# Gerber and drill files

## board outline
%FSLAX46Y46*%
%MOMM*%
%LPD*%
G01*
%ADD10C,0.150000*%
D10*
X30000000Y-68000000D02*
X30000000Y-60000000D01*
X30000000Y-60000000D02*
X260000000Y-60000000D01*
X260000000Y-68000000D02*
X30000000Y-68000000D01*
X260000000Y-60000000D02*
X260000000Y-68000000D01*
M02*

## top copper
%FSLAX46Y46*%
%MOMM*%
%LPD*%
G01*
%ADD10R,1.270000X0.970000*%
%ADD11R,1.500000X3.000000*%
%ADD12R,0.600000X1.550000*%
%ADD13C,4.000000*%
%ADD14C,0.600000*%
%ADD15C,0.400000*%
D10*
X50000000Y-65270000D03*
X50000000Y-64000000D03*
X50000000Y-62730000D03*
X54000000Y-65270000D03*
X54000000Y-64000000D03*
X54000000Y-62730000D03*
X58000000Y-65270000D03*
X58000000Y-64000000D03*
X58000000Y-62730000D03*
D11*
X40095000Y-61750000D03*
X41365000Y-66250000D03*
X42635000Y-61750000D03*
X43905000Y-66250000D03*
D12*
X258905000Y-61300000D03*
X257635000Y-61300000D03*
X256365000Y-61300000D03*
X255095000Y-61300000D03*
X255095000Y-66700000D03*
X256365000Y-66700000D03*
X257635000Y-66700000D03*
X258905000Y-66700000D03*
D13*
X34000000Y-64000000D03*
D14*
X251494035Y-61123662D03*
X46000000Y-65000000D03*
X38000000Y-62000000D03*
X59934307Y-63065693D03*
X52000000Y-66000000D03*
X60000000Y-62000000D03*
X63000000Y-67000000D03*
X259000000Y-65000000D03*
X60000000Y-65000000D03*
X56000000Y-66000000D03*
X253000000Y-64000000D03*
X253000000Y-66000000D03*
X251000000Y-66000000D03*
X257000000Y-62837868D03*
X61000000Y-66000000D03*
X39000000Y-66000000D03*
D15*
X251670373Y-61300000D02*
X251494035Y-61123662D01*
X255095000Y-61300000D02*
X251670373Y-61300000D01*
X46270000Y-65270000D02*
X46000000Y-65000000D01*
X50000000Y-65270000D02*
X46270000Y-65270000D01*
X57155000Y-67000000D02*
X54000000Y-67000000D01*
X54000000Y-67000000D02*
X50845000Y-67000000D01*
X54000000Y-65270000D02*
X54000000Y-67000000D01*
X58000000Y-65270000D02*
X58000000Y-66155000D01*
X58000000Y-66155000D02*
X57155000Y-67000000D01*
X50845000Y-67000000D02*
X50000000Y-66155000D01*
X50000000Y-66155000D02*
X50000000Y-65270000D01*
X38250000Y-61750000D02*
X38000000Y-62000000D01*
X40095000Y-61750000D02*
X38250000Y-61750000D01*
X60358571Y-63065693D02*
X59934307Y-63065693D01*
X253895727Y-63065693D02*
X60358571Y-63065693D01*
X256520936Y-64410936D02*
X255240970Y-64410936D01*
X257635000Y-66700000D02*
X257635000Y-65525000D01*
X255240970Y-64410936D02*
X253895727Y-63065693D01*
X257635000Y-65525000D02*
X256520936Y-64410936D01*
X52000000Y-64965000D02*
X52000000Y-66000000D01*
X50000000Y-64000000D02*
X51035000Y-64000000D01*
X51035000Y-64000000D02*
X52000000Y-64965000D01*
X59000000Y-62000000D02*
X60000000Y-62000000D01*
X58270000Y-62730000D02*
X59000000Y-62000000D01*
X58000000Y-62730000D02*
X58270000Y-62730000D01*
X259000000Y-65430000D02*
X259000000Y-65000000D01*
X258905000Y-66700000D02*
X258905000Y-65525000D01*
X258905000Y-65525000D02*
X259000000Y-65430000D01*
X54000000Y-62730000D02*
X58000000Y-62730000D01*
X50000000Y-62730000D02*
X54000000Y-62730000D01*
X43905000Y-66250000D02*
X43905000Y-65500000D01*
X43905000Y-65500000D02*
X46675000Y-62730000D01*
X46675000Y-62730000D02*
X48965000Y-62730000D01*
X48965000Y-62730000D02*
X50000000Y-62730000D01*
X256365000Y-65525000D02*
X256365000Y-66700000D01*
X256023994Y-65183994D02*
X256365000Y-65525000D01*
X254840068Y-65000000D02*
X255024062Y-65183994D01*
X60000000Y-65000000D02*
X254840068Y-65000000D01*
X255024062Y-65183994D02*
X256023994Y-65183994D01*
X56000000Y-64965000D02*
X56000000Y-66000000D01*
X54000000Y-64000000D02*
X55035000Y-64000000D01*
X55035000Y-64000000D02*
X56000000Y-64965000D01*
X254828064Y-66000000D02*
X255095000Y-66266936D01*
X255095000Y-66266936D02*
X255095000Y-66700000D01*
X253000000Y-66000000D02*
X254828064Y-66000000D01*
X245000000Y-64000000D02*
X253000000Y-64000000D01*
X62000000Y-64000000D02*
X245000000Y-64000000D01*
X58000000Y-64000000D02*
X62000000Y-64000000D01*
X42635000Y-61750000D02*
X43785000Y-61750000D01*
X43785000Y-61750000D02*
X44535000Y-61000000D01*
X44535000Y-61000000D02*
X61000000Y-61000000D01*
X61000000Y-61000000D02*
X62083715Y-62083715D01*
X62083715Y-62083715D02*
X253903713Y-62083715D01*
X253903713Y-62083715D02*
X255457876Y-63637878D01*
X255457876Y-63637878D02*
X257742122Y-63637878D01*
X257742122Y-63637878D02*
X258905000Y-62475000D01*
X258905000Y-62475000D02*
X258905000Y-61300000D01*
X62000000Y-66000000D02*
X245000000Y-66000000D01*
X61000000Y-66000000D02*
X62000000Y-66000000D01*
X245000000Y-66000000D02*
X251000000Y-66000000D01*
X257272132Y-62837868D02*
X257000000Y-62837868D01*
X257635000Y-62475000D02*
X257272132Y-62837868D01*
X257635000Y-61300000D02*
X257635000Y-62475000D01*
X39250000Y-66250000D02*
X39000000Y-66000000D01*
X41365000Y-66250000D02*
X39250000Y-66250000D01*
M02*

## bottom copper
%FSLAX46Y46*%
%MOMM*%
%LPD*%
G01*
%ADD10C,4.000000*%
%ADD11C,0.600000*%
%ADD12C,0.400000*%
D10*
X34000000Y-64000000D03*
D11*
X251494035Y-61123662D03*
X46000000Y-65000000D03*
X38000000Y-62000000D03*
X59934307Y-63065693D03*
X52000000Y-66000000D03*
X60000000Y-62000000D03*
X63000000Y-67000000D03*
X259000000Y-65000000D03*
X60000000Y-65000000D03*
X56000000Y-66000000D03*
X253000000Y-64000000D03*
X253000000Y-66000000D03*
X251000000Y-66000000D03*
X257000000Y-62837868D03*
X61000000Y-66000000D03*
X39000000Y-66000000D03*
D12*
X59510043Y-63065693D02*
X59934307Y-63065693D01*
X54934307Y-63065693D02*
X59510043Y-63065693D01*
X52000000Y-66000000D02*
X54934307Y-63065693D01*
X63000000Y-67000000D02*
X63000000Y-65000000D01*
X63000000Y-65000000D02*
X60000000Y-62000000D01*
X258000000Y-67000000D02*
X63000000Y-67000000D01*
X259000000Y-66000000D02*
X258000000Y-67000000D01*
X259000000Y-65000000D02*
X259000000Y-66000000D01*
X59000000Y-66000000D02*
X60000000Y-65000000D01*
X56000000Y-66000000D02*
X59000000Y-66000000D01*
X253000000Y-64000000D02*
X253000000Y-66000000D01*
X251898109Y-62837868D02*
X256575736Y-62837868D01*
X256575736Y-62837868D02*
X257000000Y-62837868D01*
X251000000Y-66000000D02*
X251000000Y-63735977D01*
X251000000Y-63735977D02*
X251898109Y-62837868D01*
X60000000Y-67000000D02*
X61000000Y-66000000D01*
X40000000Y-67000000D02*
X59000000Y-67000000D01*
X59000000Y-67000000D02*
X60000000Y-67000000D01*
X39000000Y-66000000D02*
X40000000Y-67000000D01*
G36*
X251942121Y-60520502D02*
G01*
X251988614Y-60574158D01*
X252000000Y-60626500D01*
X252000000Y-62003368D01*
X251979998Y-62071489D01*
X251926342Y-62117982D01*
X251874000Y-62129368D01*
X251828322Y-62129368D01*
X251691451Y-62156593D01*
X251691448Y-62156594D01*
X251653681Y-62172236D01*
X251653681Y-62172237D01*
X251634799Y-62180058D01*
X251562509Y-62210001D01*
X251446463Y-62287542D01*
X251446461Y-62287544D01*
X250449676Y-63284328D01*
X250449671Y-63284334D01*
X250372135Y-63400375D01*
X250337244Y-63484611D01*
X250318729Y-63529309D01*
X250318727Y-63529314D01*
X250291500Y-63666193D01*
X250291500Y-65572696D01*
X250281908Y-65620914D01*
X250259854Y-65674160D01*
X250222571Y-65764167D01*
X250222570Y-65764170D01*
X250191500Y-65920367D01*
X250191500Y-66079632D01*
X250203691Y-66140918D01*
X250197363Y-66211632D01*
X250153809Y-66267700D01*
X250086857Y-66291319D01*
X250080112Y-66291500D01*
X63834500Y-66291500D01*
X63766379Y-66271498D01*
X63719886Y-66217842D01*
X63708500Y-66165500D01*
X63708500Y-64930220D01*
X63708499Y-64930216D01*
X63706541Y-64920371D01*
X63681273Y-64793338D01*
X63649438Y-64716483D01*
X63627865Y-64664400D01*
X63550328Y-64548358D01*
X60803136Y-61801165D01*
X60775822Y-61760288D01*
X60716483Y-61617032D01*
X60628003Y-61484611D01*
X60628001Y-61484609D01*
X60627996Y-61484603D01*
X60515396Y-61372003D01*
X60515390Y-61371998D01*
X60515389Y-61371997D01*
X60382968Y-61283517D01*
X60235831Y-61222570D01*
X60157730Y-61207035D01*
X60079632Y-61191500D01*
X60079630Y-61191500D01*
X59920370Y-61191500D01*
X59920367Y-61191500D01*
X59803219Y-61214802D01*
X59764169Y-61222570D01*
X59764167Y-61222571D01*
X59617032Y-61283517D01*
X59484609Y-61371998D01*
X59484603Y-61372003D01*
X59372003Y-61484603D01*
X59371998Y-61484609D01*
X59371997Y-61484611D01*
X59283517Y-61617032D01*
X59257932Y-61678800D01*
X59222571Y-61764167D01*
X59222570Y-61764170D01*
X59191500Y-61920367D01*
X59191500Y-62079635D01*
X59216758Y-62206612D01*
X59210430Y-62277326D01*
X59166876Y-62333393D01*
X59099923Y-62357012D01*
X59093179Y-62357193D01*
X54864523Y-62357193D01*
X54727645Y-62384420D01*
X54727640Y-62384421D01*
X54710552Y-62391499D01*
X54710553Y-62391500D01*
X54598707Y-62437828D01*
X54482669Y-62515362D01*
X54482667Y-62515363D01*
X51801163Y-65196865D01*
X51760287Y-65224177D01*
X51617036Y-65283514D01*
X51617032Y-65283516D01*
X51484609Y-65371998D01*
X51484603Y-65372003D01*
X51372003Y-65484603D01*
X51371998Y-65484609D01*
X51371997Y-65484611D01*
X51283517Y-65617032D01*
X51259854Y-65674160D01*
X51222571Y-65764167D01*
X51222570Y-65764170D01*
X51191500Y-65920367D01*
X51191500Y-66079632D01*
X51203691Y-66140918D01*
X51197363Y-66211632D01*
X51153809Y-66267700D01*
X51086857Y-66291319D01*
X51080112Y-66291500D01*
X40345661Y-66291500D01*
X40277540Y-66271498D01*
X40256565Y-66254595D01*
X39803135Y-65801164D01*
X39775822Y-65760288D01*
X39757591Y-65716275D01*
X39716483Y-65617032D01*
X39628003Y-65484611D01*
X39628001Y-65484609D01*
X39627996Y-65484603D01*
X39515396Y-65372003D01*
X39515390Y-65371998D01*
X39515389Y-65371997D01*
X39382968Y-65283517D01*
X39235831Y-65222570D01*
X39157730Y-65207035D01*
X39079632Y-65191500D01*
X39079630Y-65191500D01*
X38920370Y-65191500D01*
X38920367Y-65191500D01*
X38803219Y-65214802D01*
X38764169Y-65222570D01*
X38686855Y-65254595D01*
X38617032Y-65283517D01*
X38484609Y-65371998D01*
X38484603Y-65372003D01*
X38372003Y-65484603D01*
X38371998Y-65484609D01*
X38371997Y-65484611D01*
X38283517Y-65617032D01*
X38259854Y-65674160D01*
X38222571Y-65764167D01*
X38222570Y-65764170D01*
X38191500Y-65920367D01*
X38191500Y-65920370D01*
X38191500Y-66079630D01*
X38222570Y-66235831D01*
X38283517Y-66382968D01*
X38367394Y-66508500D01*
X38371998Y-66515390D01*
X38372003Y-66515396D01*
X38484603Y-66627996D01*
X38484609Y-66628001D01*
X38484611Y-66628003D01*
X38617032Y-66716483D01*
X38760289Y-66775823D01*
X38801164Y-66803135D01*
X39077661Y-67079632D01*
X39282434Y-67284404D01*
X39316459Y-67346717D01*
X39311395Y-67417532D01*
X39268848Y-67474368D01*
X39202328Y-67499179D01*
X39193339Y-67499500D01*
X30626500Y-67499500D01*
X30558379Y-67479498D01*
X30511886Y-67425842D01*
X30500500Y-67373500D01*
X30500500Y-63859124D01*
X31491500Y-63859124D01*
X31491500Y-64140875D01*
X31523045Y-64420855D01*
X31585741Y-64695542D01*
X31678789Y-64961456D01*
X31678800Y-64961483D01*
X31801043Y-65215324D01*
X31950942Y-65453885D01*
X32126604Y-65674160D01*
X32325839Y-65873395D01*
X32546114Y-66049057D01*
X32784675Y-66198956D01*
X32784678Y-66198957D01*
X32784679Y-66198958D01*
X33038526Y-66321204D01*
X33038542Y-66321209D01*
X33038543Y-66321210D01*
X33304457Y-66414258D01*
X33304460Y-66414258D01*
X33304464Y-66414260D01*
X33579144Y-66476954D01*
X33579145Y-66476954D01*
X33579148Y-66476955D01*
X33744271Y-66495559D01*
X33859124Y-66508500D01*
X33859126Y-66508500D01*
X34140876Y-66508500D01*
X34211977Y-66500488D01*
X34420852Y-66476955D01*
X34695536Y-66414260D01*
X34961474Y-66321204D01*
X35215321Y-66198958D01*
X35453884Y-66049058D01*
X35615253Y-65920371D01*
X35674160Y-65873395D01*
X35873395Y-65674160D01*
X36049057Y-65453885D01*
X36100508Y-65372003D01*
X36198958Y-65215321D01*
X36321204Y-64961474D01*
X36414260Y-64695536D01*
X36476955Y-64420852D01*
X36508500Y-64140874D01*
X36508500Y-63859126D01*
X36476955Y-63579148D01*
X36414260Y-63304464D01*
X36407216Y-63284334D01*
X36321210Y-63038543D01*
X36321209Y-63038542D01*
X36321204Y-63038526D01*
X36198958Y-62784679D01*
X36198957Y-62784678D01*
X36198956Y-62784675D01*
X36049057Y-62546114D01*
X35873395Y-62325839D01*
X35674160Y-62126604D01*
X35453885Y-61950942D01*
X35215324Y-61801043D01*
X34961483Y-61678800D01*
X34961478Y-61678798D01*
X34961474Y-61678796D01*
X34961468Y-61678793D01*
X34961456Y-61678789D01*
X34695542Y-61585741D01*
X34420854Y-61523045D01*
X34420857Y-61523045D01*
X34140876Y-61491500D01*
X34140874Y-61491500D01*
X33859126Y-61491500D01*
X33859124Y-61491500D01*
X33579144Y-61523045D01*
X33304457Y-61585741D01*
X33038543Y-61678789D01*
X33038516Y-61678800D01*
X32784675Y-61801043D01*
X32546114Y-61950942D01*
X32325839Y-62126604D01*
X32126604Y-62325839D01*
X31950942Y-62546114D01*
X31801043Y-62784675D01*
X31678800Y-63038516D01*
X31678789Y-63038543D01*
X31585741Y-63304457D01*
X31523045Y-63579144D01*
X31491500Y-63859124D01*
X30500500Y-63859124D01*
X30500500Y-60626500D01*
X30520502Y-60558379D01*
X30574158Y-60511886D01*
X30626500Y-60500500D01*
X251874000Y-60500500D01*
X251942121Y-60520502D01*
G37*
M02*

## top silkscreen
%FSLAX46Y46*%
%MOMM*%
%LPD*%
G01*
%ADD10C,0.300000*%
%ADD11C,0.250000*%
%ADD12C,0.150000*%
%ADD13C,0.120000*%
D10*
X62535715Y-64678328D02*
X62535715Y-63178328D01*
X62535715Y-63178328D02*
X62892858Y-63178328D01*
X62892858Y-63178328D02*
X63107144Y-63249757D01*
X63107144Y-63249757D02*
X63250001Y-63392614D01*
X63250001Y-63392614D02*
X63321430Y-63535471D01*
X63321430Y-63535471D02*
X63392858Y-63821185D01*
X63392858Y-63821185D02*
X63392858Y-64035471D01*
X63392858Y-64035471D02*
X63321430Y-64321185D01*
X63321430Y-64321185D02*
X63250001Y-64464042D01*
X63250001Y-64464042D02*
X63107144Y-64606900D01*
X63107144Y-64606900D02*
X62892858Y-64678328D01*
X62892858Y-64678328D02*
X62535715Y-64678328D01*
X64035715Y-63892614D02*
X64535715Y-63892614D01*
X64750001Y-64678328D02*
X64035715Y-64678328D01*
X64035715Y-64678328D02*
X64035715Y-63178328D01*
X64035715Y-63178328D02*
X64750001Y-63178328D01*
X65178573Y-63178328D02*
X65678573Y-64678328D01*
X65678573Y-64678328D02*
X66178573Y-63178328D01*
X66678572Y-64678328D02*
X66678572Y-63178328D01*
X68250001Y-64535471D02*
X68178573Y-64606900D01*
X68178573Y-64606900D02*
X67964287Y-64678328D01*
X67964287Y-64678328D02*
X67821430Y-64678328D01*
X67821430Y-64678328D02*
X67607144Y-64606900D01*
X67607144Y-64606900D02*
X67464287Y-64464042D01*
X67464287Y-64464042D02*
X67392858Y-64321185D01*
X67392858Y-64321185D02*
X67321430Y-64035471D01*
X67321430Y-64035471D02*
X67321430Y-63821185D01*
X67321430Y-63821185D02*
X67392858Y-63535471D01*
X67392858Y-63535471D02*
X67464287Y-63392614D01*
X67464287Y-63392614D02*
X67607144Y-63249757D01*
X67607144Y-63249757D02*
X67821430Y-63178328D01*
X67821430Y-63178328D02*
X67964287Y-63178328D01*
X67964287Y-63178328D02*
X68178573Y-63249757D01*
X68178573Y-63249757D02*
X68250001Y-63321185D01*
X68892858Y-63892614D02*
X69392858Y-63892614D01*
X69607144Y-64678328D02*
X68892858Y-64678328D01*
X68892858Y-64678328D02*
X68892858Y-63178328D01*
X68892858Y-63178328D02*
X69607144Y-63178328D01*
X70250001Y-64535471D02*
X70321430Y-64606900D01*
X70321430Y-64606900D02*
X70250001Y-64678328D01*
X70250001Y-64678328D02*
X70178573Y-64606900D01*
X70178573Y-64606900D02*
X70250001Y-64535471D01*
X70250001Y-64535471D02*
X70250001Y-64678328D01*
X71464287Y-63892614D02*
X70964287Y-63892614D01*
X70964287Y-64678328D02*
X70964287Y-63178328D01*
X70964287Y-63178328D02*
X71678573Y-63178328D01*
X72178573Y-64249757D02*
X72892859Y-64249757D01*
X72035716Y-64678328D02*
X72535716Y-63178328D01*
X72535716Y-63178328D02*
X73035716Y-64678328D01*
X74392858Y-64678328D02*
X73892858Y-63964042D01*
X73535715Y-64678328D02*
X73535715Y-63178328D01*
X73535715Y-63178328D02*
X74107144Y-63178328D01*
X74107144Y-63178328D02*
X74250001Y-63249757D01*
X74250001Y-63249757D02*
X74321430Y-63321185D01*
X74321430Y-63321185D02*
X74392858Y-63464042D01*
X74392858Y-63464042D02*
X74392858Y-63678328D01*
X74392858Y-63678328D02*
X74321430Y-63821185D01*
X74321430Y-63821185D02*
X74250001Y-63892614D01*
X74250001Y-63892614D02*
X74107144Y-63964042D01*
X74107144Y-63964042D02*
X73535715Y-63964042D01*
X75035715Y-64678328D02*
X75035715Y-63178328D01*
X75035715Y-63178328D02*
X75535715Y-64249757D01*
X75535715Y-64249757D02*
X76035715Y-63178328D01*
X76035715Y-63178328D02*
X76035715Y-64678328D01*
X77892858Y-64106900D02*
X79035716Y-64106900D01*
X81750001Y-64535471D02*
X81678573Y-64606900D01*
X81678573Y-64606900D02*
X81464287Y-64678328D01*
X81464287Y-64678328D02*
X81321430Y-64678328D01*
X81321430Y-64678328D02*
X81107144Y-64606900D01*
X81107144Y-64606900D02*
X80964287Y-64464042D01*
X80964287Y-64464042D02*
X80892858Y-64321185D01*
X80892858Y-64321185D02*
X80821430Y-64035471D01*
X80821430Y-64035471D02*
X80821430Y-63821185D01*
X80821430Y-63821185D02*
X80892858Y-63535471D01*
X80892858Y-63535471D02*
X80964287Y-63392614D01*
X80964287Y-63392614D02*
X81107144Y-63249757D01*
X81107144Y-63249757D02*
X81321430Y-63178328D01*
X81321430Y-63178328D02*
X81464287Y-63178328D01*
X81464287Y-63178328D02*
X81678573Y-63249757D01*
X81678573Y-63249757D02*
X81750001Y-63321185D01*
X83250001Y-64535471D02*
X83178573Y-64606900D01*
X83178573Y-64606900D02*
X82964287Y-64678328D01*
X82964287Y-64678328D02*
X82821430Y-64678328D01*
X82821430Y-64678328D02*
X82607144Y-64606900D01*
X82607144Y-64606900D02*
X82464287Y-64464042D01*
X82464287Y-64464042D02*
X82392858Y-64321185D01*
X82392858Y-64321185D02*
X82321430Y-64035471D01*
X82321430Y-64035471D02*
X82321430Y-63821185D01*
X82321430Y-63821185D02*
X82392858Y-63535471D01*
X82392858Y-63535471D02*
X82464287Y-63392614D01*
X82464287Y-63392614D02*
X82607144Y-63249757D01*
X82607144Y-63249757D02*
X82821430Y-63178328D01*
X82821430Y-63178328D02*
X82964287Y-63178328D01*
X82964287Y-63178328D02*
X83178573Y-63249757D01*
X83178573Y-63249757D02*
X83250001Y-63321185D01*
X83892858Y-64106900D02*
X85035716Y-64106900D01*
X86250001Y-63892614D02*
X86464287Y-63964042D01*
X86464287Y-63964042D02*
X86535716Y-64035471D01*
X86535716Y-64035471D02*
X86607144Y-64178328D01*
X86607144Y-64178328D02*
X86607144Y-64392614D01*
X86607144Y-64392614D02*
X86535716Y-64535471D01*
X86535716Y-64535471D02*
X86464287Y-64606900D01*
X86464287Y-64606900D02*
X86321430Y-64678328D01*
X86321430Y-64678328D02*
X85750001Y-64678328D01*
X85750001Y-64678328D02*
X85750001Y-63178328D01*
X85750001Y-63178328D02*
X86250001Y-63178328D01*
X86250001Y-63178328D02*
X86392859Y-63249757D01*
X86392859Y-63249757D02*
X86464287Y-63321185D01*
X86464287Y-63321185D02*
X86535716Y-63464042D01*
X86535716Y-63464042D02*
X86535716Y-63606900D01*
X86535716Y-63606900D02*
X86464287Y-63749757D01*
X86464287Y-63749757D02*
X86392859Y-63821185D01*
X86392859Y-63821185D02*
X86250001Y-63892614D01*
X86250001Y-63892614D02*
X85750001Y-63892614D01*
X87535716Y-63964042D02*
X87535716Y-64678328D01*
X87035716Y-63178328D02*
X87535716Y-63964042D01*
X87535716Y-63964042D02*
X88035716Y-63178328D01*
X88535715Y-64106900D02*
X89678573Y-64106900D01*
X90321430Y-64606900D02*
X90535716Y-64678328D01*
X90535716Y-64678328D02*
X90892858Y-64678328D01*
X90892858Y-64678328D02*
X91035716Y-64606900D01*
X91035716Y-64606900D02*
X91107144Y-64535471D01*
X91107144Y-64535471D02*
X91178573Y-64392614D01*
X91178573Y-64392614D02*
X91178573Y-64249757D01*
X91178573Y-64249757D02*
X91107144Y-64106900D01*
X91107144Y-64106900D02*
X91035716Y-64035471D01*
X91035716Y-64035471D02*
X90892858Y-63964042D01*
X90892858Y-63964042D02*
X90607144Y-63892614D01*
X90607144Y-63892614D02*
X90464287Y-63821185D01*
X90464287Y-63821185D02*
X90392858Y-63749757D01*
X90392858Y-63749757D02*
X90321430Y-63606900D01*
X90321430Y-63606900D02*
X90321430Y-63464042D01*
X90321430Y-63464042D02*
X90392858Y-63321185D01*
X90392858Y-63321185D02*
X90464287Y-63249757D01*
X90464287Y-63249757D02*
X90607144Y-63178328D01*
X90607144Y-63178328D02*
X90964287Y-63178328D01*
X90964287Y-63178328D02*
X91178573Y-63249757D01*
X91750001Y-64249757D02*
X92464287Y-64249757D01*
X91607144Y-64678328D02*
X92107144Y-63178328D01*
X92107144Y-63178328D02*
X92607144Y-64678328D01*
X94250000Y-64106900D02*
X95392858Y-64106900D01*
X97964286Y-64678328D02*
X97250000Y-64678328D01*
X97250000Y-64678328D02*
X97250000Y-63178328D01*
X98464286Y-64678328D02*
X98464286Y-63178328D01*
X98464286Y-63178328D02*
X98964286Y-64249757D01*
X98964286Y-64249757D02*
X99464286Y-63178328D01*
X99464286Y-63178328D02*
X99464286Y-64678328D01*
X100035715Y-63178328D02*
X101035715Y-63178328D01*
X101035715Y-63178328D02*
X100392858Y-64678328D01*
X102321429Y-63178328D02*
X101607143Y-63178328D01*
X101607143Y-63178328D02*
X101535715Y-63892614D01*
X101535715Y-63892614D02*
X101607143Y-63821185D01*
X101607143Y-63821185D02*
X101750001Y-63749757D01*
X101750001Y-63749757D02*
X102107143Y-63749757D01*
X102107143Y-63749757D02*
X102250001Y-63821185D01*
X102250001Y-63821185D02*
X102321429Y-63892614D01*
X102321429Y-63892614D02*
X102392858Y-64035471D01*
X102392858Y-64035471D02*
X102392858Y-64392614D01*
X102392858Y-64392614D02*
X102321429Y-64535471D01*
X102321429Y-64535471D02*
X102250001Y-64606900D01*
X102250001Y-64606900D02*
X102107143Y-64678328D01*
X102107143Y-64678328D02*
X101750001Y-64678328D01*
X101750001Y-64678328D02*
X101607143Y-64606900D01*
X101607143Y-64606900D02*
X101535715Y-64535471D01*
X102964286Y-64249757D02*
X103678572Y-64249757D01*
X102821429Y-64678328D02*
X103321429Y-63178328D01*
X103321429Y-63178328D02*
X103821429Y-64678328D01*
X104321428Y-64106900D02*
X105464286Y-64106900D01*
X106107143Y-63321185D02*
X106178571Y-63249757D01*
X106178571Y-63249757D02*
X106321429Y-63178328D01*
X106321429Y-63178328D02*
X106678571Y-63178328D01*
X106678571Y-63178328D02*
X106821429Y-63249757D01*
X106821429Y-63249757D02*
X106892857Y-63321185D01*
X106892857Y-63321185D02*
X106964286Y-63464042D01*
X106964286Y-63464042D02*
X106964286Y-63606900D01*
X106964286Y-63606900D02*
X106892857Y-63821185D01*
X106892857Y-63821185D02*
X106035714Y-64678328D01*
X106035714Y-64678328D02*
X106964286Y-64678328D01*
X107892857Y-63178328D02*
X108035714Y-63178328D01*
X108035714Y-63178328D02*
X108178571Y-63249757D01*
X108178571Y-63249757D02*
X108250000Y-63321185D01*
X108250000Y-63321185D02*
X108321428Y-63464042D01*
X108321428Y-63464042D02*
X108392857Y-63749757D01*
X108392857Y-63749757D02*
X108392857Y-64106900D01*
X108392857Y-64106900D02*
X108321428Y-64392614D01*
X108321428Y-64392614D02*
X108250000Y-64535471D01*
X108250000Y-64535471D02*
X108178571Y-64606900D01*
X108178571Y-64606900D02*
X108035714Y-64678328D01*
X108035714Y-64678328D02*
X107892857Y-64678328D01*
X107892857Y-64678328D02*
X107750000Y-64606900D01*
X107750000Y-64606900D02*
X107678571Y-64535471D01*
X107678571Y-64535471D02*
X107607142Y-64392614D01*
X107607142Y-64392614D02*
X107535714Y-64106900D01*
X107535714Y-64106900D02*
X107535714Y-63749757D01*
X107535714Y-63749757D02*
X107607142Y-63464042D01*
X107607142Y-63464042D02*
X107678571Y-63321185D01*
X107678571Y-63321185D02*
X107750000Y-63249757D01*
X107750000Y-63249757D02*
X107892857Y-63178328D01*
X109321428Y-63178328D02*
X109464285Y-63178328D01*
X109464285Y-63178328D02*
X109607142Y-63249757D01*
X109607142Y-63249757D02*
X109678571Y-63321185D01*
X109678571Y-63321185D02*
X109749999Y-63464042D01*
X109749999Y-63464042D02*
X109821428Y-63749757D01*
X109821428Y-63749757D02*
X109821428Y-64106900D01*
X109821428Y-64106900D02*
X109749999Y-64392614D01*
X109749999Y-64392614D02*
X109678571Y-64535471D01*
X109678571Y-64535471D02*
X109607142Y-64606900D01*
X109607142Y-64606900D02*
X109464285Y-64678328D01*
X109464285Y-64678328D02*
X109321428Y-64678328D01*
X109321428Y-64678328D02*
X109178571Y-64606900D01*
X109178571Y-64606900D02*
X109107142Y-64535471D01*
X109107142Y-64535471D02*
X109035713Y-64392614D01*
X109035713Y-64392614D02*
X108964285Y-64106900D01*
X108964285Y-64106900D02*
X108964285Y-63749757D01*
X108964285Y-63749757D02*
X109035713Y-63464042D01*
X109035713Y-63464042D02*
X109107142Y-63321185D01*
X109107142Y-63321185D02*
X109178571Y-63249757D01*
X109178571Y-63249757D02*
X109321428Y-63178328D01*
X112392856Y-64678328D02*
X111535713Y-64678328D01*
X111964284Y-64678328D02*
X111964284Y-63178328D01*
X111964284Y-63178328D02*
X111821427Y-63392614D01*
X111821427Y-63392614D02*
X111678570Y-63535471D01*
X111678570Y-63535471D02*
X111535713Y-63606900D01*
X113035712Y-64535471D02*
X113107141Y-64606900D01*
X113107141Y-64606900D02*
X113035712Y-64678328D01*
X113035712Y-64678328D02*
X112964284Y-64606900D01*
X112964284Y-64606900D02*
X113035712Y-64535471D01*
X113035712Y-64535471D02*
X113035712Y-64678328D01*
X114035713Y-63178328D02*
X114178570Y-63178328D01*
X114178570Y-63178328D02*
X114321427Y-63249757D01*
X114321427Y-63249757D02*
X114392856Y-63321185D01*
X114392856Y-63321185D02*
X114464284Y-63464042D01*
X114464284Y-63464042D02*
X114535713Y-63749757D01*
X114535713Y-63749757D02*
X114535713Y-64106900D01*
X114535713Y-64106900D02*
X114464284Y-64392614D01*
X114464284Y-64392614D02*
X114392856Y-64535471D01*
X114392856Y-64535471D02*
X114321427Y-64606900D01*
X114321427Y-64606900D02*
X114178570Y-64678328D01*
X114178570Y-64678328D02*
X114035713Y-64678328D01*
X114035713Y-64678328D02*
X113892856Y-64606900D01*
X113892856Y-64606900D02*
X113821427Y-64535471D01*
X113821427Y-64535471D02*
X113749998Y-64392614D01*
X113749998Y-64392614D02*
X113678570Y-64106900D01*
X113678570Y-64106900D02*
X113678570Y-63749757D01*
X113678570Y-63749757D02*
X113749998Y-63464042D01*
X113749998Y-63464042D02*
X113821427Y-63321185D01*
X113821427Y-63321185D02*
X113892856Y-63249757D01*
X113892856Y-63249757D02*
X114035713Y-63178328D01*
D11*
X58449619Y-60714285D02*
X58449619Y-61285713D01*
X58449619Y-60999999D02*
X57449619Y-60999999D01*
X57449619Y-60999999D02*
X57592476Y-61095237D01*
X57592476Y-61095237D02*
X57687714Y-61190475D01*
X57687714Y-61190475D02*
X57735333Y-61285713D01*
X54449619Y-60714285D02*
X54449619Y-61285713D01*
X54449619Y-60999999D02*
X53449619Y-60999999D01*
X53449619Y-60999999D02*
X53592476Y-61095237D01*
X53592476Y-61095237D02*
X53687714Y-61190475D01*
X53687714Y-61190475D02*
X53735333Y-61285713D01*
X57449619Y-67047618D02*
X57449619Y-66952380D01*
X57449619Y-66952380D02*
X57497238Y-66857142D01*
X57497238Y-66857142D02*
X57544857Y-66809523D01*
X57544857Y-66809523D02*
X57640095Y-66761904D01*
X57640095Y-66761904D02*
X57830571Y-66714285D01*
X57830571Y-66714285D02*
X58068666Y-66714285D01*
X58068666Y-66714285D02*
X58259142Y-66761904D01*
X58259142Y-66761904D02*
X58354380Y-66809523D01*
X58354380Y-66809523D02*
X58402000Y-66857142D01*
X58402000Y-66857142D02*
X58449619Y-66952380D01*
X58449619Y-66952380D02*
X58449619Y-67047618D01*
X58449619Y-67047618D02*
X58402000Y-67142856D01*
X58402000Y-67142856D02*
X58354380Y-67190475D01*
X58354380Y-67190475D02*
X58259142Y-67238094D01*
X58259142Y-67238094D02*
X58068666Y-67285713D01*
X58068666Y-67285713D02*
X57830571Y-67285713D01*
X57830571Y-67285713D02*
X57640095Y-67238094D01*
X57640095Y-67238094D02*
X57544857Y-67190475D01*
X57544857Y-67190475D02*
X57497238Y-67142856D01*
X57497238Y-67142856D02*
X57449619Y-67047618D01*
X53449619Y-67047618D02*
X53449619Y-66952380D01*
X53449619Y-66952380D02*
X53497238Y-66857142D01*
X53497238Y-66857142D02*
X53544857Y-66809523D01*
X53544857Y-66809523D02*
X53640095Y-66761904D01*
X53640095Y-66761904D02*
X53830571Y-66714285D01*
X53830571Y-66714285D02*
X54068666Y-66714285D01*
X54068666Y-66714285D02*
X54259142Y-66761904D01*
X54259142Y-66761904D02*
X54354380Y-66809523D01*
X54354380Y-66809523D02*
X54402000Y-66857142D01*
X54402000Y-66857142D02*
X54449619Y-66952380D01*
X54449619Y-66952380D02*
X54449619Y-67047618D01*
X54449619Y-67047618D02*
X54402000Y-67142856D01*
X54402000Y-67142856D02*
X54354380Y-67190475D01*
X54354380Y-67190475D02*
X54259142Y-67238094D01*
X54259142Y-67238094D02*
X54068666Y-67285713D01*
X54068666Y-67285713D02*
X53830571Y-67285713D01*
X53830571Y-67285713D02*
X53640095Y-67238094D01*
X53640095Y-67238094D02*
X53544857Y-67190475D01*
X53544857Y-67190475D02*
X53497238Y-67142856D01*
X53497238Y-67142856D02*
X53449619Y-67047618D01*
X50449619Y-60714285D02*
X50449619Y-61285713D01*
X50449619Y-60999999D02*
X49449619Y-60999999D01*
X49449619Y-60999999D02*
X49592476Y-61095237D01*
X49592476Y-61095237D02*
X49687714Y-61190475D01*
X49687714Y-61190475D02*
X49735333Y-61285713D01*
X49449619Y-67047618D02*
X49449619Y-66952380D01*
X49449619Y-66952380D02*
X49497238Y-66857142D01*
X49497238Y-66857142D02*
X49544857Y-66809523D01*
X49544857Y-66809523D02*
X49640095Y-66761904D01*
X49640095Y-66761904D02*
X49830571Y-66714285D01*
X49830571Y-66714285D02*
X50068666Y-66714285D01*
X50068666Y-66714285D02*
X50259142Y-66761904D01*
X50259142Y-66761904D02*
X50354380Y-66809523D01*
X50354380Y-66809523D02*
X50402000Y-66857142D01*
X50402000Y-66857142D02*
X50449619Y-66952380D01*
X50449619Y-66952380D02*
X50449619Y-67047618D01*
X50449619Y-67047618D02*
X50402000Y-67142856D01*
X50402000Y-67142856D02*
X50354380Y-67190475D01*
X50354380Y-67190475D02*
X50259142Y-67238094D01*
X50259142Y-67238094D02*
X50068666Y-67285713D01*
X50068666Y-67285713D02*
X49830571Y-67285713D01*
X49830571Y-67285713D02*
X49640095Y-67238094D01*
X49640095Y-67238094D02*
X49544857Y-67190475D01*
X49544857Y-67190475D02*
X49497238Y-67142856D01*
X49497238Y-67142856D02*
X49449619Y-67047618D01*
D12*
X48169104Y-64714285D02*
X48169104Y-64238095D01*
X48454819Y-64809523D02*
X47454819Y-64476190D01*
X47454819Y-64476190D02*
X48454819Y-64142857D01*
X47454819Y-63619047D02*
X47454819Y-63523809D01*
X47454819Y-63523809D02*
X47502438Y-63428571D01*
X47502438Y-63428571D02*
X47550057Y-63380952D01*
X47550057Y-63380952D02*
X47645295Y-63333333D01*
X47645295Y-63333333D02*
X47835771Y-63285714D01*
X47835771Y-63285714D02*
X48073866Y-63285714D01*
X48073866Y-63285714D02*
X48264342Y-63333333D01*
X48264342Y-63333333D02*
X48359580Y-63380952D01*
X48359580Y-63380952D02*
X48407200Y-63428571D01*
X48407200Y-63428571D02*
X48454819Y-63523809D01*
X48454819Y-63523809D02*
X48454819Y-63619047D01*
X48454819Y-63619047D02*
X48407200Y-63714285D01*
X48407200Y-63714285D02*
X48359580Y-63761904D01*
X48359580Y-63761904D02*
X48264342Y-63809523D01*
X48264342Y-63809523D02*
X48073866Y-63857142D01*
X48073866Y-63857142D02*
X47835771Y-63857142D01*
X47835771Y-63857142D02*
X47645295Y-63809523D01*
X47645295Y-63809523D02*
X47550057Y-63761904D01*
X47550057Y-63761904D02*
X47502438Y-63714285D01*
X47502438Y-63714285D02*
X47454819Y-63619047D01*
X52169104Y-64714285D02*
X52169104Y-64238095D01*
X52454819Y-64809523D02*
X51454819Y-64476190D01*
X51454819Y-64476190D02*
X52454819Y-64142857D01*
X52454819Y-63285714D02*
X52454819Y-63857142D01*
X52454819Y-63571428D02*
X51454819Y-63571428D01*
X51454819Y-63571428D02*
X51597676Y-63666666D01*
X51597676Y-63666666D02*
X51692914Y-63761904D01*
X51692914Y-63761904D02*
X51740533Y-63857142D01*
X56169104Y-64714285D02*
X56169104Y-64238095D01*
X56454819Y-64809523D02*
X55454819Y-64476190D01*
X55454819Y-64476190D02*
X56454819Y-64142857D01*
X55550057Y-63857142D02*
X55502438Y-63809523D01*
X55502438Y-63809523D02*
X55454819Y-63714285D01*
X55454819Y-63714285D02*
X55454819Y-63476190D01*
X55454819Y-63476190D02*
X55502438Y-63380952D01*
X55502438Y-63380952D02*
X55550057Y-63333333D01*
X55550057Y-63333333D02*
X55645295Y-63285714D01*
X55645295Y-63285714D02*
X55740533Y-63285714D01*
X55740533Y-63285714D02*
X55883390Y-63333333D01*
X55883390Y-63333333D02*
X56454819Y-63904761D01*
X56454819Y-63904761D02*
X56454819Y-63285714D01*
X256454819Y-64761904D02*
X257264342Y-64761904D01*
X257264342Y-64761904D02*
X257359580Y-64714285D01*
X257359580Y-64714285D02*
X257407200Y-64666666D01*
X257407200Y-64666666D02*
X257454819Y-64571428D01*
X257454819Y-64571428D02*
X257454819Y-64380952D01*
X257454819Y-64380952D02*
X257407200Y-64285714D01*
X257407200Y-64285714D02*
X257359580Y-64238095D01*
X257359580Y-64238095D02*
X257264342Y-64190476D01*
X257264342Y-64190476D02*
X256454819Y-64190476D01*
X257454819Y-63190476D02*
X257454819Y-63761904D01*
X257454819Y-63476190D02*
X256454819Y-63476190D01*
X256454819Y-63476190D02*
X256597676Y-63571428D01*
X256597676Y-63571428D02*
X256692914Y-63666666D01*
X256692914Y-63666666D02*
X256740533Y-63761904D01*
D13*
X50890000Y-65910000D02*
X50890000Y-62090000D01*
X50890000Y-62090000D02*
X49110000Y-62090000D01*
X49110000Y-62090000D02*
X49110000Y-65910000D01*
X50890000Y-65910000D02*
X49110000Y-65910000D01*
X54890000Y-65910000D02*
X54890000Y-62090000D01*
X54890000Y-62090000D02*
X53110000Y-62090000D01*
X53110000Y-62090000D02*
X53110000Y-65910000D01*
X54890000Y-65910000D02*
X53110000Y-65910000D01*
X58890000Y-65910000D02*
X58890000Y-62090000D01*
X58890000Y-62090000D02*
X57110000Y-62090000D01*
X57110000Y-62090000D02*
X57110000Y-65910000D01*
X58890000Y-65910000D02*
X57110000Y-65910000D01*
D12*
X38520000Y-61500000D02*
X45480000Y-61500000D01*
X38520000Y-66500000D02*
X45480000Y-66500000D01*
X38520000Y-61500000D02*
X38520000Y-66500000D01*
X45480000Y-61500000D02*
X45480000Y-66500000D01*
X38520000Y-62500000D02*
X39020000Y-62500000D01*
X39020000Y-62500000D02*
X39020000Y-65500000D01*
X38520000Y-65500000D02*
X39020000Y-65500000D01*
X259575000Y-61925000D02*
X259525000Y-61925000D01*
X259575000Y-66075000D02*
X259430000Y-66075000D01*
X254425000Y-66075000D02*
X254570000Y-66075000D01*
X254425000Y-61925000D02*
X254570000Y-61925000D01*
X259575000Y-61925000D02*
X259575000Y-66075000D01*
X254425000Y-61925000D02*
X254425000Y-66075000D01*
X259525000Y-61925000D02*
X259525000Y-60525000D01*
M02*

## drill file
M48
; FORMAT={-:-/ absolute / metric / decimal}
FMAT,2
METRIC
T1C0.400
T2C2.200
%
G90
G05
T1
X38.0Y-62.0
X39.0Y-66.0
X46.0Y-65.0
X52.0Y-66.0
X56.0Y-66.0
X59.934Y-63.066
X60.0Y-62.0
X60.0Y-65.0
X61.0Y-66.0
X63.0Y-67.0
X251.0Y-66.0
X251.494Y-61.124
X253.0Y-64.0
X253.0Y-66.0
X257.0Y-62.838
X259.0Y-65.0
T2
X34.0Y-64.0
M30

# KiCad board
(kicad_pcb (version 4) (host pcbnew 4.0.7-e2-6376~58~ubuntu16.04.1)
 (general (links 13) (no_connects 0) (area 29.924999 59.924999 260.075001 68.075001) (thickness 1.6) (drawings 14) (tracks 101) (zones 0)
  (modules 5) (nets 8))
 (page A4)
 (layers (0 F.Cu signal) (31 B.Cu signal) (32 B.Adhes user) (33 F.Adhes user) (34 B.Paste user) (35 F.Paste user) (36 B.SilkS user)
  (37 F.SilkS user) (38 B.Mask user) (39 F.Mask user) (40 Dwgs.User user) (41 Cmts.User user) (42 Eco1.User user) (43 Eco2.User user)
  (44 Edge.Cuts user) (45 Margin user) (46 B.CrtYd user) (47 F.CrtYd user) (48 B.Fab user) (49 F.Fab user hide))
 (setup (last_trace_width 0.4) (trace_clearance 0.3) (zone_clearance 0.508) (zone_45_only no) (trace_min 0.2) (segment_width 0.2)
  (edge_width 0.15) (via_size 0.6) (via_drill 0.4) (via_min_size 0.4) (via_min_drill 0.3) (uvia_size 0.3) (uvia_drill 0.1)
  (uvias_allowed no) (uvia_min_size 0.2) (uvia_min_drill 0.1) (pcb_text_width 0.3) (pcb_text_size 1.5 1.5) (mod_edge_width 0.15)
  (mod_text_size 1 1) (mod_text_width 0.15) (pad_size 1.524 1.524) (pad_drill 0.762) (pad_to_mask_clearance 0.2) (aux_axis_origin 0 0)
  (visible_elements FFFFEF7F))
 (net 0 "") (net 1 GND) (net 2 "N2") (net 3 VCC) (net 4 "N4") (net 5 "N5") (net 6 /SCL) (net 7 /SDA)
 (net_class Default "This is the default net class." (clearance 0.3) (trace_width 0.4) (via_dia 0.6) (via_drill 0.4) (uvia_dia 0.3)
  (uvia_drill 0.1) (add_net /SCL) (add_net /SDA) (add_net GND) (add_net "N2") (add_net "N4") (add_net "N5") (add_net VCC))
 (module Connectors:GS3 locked (layer F.Cu) (at 50 64 180)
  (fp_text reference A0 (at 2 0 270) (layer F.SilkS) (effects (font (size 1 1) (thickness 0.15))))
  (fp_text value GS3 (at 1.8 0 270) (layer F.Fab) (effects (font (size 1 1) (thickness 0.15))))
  (fp_line (start -0.89 -1.91) (end -0.89 1.91) (layer F.SilkS) (width 0.12))
  (fp_line (start -0.89 1.91) (end 0.89 1.91) (layer F.SilkS) (width 0.12))
  (fp_line (start 0.89 1.91) (end 0.89 -1.91) (layer F.SilkS) (width 0.12))
  (fp_line (start -0.89 -1.91) (end 0.89 -1.91) (layer F.SilkS) (width 0.12))
  (pad 1 smd rect (at 0 -1.27 180) (size 1.27 0.97) (layers F.Cu F.Paste F.Mask) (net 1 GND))
  (pad 2 smd rect (at 0 0 180) (size 1.27 0.97) (layers F.Cu F.Paste F.Mask) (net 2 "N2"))
  (pad 3 smd rect (at 0 1.27 180) (size 1.27 0.97) (layers F.Cu F.Paste F.Mask) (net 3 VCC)))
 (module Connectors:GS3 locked (layer F.Cu) (at 54 64 180)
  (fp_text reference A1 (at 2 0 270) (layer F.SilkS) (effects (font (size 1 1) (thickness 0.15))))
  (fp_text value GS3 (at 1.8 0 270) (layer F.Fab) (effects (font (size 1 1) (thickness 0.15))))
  (fp_line (start -0.89 -1.91) (end -0.89 1.91) (layer F.SilkS) (width 0.12))
  (fp_line (start -0.89 1.91) (end 0.89 1.91) (layer F.SilkS) (width 0.12))
  (fp_line (start 0.89 1.91) (end 0.89 -1.91) (layer F.SilkS) (width 0.12))
  (fp_line (start -0.89 -1.91) (end 0.89 -1.91) (layer F.SilkS) (width 0.12))
  (pad 1 smd rect (at 0 -1.27 180) (size 1.27 0.97) (layers F.Cu F.Paste F.Mask) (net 1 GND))
  (pad 2 smd rect (at 0 0 180) (size 1.27 0.97) (layers F.Cu F.Paste F.Mask) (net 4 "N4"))
  (pad 3 smd rect (at 0 1.27 180) (size 1.27 0.97) (layers F.Cu F.Paste F.Mask) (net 3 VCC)))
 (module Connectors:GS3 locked (layer F.Cu) (at 58 64 180)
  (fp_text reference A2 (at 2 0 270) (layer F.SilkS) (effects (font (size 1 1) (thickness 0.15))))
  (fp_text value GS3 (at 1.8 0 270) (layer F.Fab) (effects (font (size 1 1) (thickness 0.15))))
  (fp_line (start -0.89 -1.91) (end -0.89 1.91) (layer F.SilkS) (width 0.12))
  (fp_line (start -0.89 1.91) (end 0.89 1.91) (layer F.SilkS) (width 0.12))
  (fp_line (start 0.89 1.91) (end 0.89 -1.91) (layer F.SilkS) (width 0.12))
  (fp_line (start -0.89 -1.91) (end 0.89 -1.91) (layer F.SilkS) (width 0.12))
  (pad 1 smd rect (at 0 -1.27 180) (size 1.27 0.97) (layers F.Cu F.Paste F.Mask) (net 1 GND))
  (pad 2 smd rect (at 0 0 180) (size 1.27 0.97) (layers F.Cu F.Paste F.Mask) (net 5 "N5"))
  (pad 3 smd rect (at 0 1.27 180) (size 1.27 0.97) (layers F.Cu F.Paste F.Mask) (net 3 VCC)))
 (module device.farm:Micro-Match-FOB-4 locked (layer F.Cu) (at 42 64)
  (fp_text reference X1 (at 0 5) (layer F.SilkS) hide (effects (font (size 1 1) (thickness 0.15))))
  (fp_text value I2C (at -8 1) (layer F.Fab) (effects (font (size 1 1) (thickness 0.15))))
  (fp_line (start -3.48 -2.5) (end 3.48 -2.5) (layer F.SilkS) (width 0.15))
  (fp_line (start -3.48 2.5) (end 3.48 2.5) (layer F.SilkS) (width 0.15))
  (fp_line (start -3.48 -2.5) (end -3.48 2.5) (layer F.SilkS) (width 0.15))
  (fp_line (start 3.48 -2.5) (end 3.48 2.5) (layer F.SilkS) (width 0.15))
  (fp_line (start -3.48 -1.5) (end -2.98 -1.5) (layer F.SilkS) (width 0.15))
  (fp_line (start -2.98 -1.5) (end -2.98 1.5) (layer F.SilkS) (width 0.15))
  (fp_line (start -3.48 1.5) (end -2.98 1.5) (layer F.SilkS) (width 0.15))
  (pad 1 smd rect (at -1.905 -2.25) (size 1.5 3) (layers F.Cu F.Paste F.Mask) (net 1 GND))
  (pad 2 smd rect (at -0.635 2.25) (size 1.5 3) (layers F.Cu F.Paste F.Mask) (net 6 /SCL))
  (pad 3 smd rect (at 0.635 -2.25) (size 1.5 3) (layers F.Cu F.Paste F.Mask) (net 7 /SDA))
  (pad 4 smd rect (at 1.905 2.25) (size 1.5 3) (layers F.Cu F.Paste F.Mask) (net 3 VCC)))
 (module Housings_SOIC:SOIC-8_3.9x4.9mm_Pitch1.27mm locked (layer F.Cu) (at 257 64 270)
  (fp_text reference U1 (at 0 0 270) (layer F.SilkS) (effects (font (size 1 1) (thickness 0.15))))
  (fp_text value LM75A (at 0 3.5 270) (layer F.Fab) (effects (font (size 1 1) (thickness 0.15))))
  (fp_line (start -2.075 -2.575) (end -2.075 -2.525) (layer F.SilkS) (width 0.15))
  (fp_line (start 2.075 -2.575) (end 2.075 -2.43) (layer F.SilkS) (width 0.15))
  (fp_line (start 2.075 2.575) (end 2.075 2.43) (layer F.SilkS) (width 0.15))
  (fp_line (start -2.075 2.575) (end -2.075 2.43) (layer F.SilkS) (width 0.15))
  (fp_line (start -2.075 -2.575) (end 2.075 -2.575) (layer F.SilkS) (width 0.15))
  (fp_line (start -2.075 2.575) (end 2.075 2.575) (layer F.SilkS) (width 0.15))
  (fp_line (start -2.075 -2.525) (end -3.475 -2.525) (layer F.SilkS) (width 0.15))
  (pad 1 smd rect (at -2.7 -1.905 270) (size 1.55 0.6) (layers F.Cu F.Paste F.Mask) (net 7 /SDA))
  (pad 2 smd rect (at -2.7 -0.635 270) (size 1.55 0.6) (layers F.Cu F.Paste F.Mask) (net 6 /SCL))
  (pad 3 smd rect (at -2.7 0.635 270) (size 1.55 0.6) (layers F.Cu F.Paste F.Mask))
  (pad 4 smd rect (at -2.7 1.905 270) (size 1.55 0.6) (layers F.Cu F.Paste F.Mask) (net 1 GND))
  (pad 5 smd rect (at 2.7 1.905 270) (size 1.55 0.6) (layers F.Cu F.Paste F.Mask) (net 5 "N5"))
  (pad 6 smd rect (at 2.7 0.635 270) (size 1.55 0.6) (layers F.Cu F.Paste F.Mask) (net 4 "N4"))
  (pad 7 smd rect (at 2.7 -0.635 270) (size 1.55 0.6) (layers F.Cu F.Paste F.Mask) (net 2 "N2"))
  (pad 8 smd rect (at 2.7 -1.905 270) (size 1.55 0.6) (layers F.Cu F.Paste F.Mask) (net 3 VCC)))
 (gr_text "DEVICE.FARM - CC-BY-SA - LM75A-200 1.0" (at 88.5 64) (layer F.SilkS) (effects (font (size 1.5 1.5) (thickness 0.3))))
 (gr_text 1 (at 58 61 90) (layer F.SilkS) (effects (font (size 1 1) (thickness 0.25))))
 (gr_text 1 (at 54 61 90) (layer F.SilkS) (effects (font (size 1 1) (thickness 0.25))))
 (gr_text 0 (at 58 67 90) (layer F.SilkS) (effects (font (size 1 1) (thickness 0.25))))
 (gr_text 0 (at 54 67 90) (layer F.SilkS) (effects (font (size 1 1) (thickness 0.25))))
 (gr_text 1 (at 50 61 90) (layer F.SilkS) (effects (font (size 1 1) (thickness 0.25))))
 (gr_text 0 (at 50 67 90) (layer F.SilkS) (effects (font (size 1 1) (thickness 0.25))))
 (gr_line (start 30 68) (end 30 60) (layer Edge.Cuts) (width 0.15))
 (gr_line (start 30 60) (end 260 60) (layer Edge.Cuts) (width 0.15))
 (gr_line (start 260 68) (end 30 68) (layer Edge.Cuts) (width 0.15))
 (gr_line (start 260 60) (end 260 68) (layer Edge.Cuts) (width 0.15))
 (via (at 34 64) (size 4) (drill 2.2) (layers F.Cu B.Cu) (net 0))
 (segment (start 251.670373 61.3) (end 251.494035 61.123662) (width 0.4) (layer F.Cu) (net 1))
 (segment (start 255.095 61.3) (end 251.670373 61.3) (width 0.4) (layer F.Cu) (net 1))
 (via (at 251.494035 61.123662) (size 0.6) (drill 0.4) (layers F.Cu B.Cu) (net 1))
 (segment (start 46.27 65.27) (end 46 65) (width 0.4) (layer F.Cu) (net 1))
 (via (at 46 65) (size 0.6) (drill 0.4) (layers F.Cu B.Cu) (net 1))
 (segment (start 50 65.27) (end 46.27 65.27) (width 0.4) (layer F.Cu) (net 1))
 (segment (start 57.155 67) (end 54 67) (width 0.4) (layer F.Cu) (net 1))
 (segment (start 54 67) (end 50.845 67) (width 0.4) (layer F.Cu) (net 1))
 (segment (start 54 65.27) (end 54 67) (width 0.4) (layer F.Cu) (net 1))
 (segment (start 58 65.27) (end 58 66.155) (width 0.4) (layer F.Cu) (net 1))
 (segment (start 58 66.155) (end 57.155 67) (width 0.4) (layer F.Cu) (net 1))
 (segment (start 50.845 67) (end 50 66.155) (width 0.4) (layer F.Cu) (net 1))
 (segment (start 50 66.155) (end 50 65.27) (width 0.4) (layer F.Cu) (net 1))
 (segment (start 38.25 61.75) (end 38 62) (width 0.4) (layer F.Cu) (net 1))
 (via (at 38 62) (size 0.6) (drill 0.4) (layers F.Cu B.Cu) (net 1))
 (segment (start 40.095 61.75) (end 38.25 61.75) (width 0.4) (layer F.Cu) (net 1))
 (segment (start 59.510043 63.065693) (end 59.934307 63.065693) (width 0.4) (layer B.Cu) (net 2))
 (segment (start 54.934307 63.065693) (end 59.510043 63.065693) (width 0.4) (layer B.Cu) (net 2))
 (segment (start 52 66) (end 54.934307 63.065693) (width 0.4) (layer B.Cu) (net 2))
 (segment (start 60.358571 63.065693) (end 59.934307 63.065693) (width 0.4) (layer F.Cu) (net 2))
 (segment (start 253.895727 63.065693) (end 60.358571 63.065693) (width 0.4) (layer F.Cu) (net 2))
 (segment (start 256.520936 64.410936) (end 255.24097 64.410936) (width 0.4) (layer F.Cu) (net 2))
 (segment (start 257.635 66.7) (end 257.635 65.525) (width 0.4) (layer F.Cu) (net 2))
 (segment (start 255.24097 64.410936) (end 253.895727 63.065693) (width 0.4) (layer F.Cu) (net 2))
 (via (at 59.934307 63.065693) (size 0.6) (drill 0.4) (layers F.Cu B.Cu) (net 2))
 (segment (start 257.635 65.525) (end 256.520936 64.410936) (width 0.4) (layer F.Cu) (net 2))
 (via (at 52 66) (size 0.6) (drill 0.4) (layers F.Cu B.Cu) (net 2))
 (segment (start 52 64.965) (end 52 66) (width 0.4) (layer F.Cu) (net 2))
 (segment (start 50 64) (end 51.035 64) (width 0.4) (layer F.Cu) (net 2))
 (segment (start 51.035 64) (end 52 64.965) (width 0.4) (layer F.Cu) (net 2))
 (segment (start 63 67) (end 63 65) (width 0.4) (layer B.Cu) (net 3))
 (segment (start 63 65) (end 60 62) (width 0.4) (layer B.Cu) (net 3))
 (segment (start 59 62) (end 60 62) (width 0.4) (layer F.Cu) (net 3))
 (via (at 60 62) (size 0.6) (drill 0.4) (layers F.Cu B.Cu) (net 3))
 (segment (start 58.27 62.73) (end 59 62) (width 0.4) (layer F.Cu) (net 3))
 (segment (start 58 62.73) (end 58.27 62.73) (width 0.4) (layer F.Cu) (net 3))
 (segment (start 258 67) (end 63 67) (width 0.4) (layer B.Cu) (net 3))
 (via (at 63 67) (size 0.6) (drill 0.4) (layers F.Cu B.Cu) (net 3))
 (segment (start 259 66) (end 258 67) (width 0.4) (layer B.Cu) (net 3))
 (segment (start 259 65) (end 259 66) (width 0.4) (layer B.Cu) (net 3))
 (segment (start 259 65.43) (end 259 65) (width 0.4) (layer F.Cu) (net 3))
 (via (at 259 65) (size 0.6) (drill 0.4) (layers F.Cu B.Cu) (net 3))
 (segment (start 258.905 66.7) (end 258.905 65.525) (width 0.4) (layer F.Cu) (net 3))
 (segment (start 258.905 65.525) (end 259 65.43) (width 0.4) (layer F.Cu) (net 3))
 (segment (start 54 62.73) (end 58 62.73) (width 0.4) (layer F.Cu) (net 3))
 (segment (start 50 62.73) (end 54 62.73) (width 0.4) (layer F.Cu) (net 3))
 (segment (start 43.905 66.25) (end 43.905 65.5) (width 0.4) (layer F.Cu) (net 3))
 (segment (start 43.905 65.5) (end 46.675 62.73) (width 0.4) (layer F.Cu) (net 3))
 (segment (start 46.675 62.73) (end 48.965 62.73) (width 0.4) (layer F.Cu) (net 3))
 (segment (start 48.965 62.73) (end 50 62.73) (width 0.4) (layer F.Cu) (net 3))
 (segment (start 256.365 65.525) (end 256.365 66.7) (width 0.4) (layer F.Cu) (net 4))
 (segment (start 256.023994 65.183994) (end 256.365 65.525) (width 0.4) (layer F.Cu) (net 4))
 (segment (start 254.840068 65) (end 255.024062 65.183994) (width 0.4) (layer F.Cu) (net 4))
 (segment (start 60 65) (end 254.840068 65) (width 0.4) (layer F.Cu) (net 4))
 (segment (start 255.024062 65.183994) (end 256.023994 65.183994) (width 0.4) (layer F.Cu) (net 4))
 (segment (start 59 66) (end 60 65) (width 0.4) (layer B.Cu) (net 4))
 (via (at 60 65) (size 0.6) (drill 0.4) (layers F.Cu B.Cu) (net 4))
 (segment (start 56 66) (end 59 66) (width 0.4) (layer B.Cu) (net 4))
 (segment (start 56 64.965) (end 56 66) (width 0.4) (layer F.Cu) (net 4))
 (via (at 56 66) (size 0.6) (drill 0.4) (layers F.Cu B.Cu) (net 4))
 (segment (start 54 64) (end 55.035 64) (width 0.4) (layer F.Cu) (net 4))
 (segment (start 55.035 64) (end 56 64.965) (width 0.4) (layer F.Cu) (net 4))
 (segment (start 254.828064 66) (end 255.095 66.266936) (width 0.4) (layer F.Cu) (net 5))
 (segment (start 255.095 66.266936) (end 255.095 66.7) (width 0.4) (layer F.Cu) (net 5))
 (segment (start 253 66) (end 254.828064 66) (width 0.4) (layer F.Cu) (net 5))
 (via (at 253 64) (size 0.6) (drill 0.4) (layers F.Cu B.Cu) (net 5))
 (segment (start 245 64) (end 253 64) (width 0.4) (layer F.Cu) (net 5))
 (segment (start 62 64) (end 245 64) (width 0.4) (layer F.Cu) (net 5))
 (segment (start 253 64) (end 253 66) (width 0.4) (layer B.Cu) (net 5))
 (segment (start 58 64) (end 62 64) (width 0.4) (layer F.Cu) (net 5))
 (via (at 253 66) (size 0.6) (drill 0.4) (layers F.Cu B.Cu) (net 5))
 (segment (start 42.635 61.75) (end 43.785 61.75) (width 0.4) (layer F.Cu) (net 7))
 (segment (start 43.785 61.75) (end 44.535 61) (width 0.4) (layer F.Cu) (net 7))
 (segment (start 44.535 61) (end 61 61) (width 0.4) (layer F.Cu) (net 7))
 (segment (start 61 61) (end 62.083715 62.083715) (width 0.4) (layer F.Cu) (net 7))
 (segment (start 62.083715 62.083715) (end 253.903713 62.083715) (width 0.4) (layer F.Cu) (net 7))
 (segment (start 253.903713 62.083715) (end 255.457876 63.637878) (width 0.4) (layer F.Cu) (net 7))
 (segment (start 255.457876 63.637878) (end 257.742122 63.637878) (width 0.4) (layer F.Cu) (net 7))
 (segment (start 257.742122 63.637878) (end 258.905 62.475) (width 0.4) (layer F.Cu) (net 7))
 (segment (start 258.905 62.475) (end 258.905 61.3) (width 0.4) (layer F.Cu) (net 7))
 (segment (start 251.898109 62.837868) (end 256.575736 62.837868) (width 0.4) (layer B.Cu) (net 6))
 (segment (start 256.575736 62.837868) (end 257 62.837868) (width 0.4) (layer B.Cu) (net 6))
 (segment (start 251 66) (end 251 63.735977) (width 0.4) (layer B.Cu) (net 6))
 (segment (start 251 63.735977) (end 251.898109 62.837868) (width 0.4) (layer B.Cu) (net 6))
 (via (at 251 66) (size 0.6) (drill 0.4) (layers F.Cu B.Cu) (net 6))
 (segment (start 62 66) (end 245 66) (width 0.4) (layer F.Cu) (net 6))
 (segment (start 61 66) (end 62 66) (width 0.4) (layer F.Cu) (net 6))
 (segment (start 245 66) (end 251 66) (width 0.4) (layer F.Cu) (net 6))
 (segment (start 257.272132 62.837868) (end 257 62.837868) (width 0.4) (layer F.Cu) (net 6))
 (segment (start 257.635 62.475) (end 257.272132 62.837868) (width 0.4) (layer F.Cu) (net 6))
 (segment (start 257.635 61.3) (end 257.635 62.475) (width 0.4) (layer F.Cu) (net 6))
 (via (at 257 62.837868) (size 0.6) (drill 0.4) (layers F.Cu B.Cu) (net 6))
 (segment (start 60 67) (end 61 66) (width 0.4) (layer B.Cu) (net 6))
 (via (at 61 66) (size 0.6) (drill 0.4) (layers F.Cu B.Cu) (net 6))
 (segment (start 40 67) (end 59 67) (width 0.4) (layer B.Cu) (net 6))
 (segment (start 59 67) (end 60 67) (width 0.4) (layer B.Cu) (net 6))
 (segment (start 39 66) (end 40 67) (width 0.4) (layer B.Cu) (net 6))
 (segment (start 39.25 66.25) (end 39 66) (width 0.4) (layer F.Cu) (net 6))
 (via (at 39 66) (size 0.6) (drill 0.4) (layers F.Cu B.Cu) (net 6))
 (segment (start 41.365 66.25) (end 39.25 66.25) (width 0.4) (layer F.Cu) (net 6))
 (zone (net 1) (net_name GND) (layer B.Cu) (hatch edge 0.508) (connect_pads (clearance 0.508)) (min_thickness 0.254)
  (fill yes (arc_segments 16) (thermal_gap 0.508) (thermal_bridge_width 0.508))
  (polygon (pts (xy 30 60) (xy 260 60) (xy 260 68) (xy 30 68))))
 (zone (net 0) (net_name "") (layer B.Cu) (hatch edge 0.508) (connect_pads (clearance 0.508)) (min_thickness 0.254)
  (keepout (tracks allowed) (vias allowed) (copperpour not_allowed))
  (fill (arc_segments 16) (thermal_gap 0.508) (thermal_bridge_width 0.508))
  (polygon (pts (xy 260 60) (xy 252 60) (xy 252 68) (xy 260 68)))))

